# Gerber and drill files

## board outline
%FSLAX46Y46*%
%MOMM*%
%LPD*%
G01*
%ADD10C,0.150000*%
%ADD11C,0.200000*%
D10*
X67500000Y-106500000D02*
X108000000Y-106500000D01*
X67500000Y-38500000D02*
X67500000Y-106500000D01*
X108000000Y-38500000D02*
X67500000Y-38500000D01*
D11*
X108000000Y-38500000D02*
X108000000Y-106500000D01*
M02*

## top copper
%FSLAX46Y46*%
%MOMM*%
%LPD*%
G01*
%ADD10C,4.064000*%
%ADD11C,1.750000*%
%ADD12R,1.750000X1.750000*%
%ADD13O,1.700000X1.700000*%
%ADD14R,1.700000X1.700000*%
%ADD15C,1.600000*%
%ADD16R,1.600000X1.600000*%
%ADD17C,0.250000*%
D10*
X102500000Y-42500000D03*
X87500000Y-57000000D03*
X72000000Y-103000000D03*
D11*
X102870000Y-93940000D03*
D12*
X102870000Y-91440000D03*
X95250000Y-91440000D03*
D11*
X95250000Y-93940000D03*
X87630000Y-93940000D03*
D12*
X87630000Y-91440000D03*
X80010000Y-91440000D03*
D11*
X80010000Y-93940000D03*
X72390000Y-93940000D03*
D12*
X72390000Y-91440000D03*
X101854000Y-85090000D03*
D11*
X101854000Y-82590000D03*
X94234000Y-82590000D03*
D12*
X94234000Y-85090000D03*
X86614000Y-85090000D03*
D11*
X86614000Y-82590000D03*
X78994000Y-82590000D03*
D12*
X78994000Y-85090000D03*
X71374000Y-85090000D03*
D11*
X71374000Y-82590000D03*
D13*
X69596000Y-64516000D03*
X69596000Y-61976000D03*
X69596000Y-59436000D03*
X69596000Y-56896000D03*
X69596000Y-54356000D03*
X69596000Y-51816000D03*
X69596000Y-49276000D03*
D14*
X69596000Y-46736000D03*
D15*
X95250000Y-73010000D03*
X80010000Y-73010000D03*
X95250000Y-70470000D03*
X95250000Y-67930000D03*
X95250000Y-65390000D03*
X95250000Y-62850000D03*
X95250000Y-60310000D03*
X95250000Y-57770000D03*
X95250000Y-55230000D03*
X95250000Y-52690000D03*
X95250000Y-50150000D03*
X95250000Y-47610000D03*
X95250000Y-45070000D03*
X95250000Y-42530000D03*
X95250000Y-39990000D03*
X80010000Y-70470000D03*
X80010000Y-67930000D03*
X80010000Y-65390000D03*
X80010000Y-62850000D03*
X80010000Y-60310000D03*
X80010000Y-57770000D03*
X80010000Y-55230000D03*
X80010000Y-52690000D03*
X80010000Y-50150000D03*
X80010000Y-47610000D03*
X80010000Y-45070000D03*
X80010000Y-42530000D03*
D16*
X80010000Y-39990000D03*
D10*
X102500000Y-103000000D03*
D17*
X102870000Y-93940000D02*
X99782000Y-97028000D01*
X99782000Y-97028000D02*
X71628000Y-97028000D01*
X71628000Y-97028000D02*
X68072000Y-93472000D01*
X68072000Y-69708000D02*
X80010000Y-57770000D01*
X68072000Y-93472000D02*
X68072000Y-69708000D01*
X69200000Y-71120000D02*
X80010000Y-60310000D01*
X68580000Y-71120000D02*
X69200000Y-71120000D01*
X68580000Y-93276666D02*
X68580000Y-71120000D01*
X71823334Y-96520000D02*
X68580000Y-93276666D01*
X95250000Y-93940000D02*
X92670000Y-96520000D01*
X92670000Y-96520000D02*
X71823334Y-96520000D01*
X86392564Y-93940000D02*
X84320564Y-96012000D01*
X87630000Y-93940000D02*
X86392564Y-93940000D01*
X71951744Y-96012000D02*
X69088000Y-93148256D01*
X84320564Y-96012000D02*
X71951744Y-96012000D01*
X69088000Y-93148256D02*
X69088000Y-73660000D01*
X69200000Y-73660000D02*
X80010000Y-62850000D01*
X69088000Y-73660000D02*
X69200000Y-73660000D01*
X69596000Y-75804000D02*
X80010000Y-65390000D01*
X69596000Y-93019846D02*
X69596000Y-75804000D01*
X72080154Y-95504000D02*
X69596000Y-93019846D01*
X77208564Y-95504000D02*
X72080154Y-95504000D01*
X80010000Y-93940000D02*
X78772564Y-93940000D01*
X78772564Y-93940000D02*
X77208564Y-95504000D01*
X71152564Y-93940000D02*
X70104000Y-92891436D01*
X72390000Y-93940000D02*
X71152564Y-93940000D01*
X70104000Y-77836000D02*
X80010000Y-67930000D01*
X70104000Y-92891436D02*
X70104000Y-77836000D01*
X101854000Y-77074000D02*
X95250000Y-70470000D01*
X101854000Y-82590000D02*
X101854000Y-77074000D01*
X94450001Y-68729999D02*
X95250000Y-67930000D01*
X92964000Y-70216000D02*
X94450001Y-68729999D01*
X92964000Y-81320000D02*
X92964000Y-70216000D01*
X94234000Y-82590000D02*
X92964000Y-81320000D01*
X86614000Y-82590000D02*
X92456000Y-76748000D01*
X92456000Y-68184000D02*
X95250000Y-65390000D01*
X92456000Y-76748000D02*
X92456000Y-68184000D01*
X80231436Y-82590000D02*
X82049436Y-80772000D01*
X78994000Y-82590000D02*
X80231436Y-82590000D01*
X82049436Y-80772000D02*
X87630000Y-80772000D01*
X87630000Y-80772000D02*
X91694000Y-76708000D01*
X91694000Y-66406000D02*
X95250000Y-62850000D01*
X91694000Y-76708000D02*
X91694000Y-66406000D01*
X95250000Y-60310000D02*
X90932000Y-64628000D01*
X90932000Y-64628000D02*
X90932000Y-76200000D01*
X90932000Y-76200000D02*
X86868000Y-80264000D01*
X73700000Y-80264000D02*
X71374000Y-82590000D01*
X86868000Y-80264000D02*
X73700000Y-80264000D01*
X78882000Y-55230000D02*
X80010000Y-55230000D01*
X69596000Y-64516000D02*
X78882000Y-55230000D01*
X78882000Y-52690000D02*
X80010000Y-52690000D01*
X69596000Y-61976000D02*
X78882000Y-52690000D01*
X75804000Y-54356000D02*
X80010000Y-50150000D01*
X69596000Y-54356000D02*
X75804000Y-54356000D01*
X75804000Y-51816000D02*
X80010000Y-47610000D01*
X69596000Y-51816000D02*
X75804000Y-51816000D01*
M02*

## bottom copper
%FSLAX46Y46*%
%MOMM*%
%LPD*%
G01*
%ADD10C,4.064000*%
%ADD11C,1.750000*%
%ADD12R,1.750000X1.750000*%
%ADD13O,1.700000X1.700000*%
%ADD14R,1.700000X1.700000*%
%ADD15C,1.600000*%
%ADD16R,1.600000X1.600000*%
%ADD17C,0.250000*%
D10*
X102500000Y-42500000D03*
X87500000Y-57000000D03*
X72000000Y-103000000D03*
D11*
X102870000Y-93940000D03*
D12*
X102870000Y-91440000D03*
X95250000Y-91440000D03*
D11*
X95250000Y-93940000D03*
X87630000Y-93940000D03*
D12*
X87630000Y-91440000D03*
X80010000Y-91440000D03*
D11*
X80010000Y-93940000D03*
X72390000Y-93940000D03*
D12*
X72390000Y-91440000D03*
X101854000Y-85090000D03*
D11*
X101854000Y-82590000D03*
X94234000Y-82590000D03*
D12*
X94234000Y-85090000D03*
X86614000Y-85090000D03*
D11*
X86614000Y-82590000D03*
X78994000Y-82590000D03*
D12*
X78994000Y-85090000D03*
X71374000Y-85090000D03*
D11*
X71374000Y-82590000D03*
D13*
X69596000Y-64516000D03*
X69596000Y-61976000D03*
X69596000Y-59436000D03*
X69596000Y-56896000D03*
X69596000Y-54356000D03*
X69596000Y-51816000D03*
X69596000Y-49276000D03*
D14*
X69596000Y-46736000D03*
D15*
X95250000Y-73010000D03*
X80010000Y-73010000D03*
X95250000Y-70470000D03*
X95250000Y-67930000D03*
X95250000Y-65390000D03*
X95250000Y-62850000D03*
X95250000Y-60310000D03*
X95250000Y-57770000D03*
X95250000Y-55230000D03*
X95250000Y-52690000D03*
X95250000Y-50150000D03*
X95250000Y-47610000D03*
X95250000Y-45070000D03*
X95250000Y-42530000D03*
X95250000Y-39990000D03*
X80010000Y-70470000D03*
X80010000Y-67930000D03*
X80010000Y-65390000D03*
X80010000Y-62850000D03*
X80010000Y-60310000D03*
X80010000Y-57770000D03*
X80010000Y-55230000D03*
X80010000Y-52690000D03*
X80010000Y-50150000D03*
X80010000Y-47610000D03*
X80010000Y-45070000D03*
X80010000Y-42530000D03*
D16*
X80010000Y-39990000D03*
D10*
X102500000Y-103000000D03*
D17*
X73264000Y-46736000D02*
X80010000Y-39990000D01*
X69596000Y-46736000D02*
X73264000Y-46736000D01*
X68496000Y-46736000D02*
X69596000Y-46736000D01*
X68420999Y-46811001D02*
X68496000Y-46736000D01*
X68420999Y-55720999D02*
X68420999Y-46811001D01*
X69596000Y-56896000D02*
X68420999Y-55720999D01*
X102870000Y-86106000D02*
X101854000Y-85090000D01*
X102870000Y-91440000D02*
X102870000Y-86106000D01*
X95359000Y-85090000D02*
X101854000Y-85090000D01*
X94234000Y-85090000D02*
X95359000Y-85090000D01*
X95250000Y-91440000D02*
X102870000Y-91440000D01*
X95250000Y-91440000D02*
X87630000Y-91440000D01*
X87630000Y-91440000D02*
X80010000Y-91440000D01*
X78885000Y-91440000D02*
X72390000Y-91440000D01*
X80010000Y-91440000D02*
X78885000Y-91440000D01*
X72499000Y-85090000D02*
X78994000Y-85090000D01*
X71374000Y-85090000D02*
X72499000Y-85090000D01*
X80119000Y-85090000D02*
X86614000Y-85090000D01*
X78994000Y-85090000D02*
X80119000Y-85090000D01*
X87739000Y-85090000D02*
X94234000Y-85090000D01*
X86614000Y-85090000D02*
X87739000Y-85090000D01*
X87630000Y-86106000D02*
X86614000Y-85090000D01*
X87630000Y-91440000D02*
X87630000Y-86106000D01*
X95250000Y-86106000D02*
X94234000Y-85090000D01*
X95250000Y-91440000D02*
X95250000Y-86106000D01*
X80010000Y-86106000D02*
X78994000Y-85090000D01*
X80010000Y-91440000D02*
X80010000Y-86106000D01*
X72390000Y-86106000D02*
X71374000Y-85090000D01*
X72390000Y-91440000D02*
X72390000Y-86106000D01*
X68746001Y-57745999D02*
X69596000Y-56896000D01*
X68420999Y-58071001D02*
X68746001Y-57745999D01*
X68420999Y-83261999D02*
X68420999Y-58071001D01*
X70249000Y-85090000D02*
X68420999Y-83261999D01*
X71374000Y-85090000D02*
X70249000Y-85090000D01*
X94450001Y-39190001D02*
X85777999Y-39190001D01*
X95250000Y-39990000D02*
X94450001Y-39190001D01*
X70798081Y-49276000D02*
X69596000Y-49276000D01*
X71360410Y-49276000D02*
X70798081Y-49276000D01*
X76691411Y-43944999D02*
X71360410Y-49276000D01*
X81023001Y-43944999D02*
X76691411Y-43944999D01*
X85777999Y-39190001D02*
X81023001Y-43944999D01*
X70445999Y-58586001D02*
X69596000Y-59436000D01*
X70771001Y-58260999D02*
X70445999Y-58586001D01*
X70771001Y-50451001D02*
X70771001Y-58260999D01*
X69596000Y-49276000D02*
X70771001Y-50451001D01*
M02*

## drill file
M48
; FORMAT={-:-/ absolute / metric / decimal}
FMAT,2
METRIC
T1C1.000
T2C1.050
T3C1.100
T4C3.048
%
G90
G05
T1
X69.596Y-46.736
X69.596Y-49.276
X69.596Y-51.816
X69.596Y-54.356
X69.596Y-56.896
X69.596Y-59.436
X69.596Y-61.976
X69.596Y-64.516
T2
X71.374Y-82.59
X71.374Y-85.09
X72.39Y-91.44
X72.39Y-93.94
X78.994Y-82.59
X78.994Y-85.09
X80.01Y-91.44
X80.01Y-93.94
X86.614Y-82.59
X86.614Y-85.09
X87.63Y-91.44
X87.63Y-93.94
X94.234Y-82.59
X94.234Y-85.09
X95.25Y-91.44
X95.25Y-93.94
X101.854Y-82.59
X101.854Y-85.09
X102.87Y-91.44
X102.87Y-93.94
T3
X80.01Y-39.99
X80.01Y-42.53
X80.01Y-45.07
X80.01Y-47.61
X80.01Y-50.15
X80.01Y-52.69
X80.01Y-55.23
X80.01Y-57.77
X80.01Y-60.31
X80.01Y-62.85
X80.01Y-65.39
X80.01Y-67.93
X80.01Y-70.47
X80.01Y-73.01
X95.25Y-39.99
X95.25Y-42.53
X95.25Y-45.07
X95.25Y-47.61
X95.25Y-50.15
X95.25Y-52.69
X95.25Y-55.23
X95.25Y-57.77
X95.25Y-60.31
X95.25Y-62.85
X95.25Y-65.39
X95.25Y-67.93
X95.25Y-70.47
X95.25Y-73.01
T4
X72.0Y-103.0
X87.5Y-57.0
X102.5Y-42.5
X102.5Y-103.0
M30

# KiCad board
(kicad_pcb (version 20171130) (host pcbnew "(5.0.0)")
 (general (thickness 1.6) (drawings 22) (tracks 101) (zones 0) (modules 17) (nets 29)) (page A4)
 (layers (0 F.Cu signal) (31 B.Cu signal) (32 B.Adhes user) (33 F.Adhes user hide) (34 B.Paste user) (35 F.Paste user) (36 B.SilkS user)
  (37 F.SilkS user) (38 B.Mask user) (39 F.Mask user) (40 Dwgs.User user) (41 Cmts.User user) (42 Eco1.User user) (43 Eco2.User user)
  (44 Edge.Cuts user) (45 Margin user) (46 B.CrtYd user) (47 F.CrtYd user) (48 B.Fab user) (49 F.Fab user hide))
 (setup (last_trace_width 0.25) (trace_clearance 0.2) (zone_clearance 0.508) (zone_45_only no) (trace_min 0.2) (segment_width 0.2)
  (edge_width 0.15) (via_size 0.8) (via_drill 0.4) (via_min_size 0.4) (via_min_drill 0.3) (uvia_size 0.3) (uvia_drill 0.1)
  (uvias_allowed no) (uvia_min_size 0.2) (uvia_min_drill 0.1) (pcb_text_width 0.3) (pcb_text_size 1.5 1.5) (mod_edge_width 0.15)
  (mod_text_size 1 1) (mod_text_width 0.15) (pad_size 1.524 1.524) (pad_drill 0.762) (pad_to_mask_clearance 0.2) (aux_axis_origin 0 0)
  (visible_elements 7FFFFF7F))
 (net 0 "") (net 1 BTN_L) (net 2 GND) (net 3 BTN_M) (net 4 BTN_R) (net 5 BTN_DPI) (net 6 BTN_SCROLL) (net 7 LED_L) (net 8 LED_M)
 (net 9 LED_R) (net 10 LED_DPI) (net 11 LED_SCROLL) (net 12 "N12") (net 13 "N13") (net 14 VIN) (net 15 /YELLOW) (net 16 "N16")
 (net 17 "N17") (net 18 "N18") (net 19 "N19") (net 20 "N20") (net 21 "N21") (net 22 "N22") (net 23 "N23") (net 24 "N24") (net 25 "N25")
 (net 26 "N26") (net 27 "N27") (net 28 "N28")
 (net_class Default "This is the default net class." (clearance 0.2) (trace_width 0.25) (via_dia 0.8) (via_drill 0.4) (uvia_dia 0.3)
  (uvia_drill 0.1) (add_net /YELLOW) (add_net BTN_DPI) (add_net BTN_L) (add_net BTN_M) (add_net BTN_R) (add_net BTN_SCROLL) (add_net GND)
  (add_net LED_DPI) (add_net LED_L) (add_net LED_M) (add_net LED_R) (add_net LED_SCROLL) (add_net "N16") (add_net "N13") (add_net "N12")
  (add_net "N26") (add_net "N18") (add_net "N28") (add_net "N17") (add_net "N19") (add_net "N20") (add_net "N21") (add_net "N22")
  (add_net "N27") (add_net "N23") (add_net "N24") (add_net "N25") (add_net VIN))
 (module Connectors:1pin (layer F.Cu) (at 102.5 42.5 90)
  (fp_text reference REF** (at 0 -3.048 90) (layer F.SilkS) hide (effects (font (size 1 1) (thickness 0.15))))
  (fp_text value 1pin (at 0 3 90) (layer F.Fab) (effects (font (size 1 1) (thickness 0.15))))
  (pad 1 thru_hole circle (at 0 0 90) (size 4.064 4.064) (drill 3.048) (layers *.Cu *.Mask)))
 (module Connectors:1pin (layer F.Cu) (at 87.5 57 90)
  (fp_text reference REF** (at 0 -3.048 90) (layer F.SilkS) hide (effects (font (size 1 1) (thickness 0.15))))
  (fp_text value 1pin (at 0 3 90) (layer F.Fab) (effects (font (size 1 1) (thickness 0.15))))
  (pad 1 thru_hole circle (at 0 0 90) (size 4.064 4.064) (drill 3.048) (layers *.Cu *.Mask)))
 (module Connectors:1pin (layer F.Cu) (at 72 103 90)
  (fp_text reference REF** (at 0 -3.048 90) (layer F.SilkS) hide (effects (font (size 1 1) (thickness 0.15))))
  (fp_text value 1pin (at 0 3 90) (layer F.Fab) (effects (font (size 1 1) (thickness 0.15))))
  (pad 1 thru_hole circle (at 0 0 90) (size 4.064 4.064) (drill 3.048) (layers *.Cu *.Mask)))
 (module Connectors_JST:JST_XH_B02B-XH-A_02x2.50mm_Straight (layer F.Cu) (at 102.87 91.44 270)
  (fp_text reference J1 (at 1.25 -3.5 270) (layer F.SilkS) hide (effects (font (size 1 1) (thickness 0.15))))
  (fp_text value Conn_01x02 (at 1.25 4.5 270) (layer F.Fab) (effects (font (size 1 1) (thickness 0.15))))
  (pad 2 thru_hole circle (at 2.5 0 270) (size 1.75 1.75) (drill 1.05) (layers *.Cu *.Mask) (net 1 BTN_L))
  (pad 1 thru_hole rect (at 0 0 270) (size 1.75 1.75) (drill 1.05) (layers *.Cu *.Mask) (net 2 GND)))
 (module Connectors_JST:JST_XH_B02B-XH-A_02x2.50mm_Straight (layer F.Cu) (at 95.25 91.44 270)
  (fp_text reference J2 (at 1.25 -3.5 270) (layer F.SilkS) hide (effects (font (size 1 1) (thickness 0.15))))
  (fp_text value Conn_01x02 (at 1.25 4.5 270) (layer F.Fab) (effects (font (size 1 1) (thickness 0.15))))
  (pad 1 thru_hole rect (at 0 0 270) (size 1.75 1.75) (drill 1.05) (layers *.Cu *.Mask) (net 2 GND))
  (pad 2 thru_hole circle (at 2.5 0 270) (size 1.75 1.75) (drill 1.05) (layers *.Cu *.Mask) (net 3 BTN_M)))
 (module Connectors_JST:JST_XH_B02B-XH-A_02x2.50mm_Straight (layer F.Cu) (at 87.63 91.44 270)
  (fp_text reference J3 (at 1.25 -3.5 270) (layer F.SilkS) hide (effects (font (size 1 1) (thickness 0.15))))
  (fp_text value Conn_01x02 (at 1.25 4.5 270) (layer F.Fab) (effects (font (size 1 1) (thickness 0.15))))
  (pad 2 thru_hole circle (at 2.5 0 270) (size 1.75 1.75) (drill 1.05) (layers *.Cu *.Mask) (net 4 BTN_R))
  (pad 1 thru_hole rect (at 0 0 270) (size 1.75 1.75) (drill 1.05) (layers *.Cu *.Mask) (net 2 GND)))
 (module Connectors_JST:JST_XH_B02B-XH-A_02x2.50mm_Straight (layer F.Cu) (at 80.01 91.44 270)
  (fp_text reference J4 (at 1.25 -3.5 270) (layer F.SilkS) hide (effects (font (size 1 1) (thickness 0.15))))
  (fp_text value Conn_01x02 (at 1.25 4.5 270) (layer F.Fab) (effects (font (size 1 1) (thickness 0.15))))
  (pad 1 thru_hole rect (at 0 0 270) (size 1.75 1.75) (drill 1.05) (layers *.Cu *.Mask) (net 2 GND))
  (pad 2 thru_hole circle (at 2.5 0 270) (size 1.75 1.75) (drill 1.05) (layers *.Cu *.Mask) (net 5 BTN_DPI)))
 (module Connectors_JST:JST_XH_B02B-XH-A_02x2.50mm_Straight (layer F.Cu) (at 72.39 91.44 270)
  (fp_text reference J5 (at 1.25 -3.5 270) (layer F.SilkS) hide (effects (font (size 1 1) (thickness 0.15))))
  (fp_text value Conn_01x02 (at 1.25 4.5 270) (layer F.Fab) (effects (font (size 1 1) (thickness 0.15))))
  (pad 2 thru_hole circle (at 2.5 0 270) (size 1.75 1.75) (drill 1.05) (layers *.Cu *.Mask) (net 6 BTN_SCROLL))
  (pad 1 thru_hole rect (at 0 0 270) (size 1.75 1.75) (drill 1.05) (layers *.Cu *.Mask) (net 2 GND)))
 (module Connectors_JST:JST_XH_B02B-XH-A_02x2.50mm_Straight (layer F.Cu) (at 101.854 85.09 90)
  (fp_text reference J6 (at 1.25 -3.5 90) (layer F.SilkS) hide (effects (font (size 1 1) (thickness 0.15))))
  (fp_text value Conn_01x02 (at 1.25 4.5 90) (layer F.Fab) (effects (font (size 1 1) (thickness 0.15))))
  (pad 1 thru_hole rect (at 0 0 90) (size 1.75 1.75) (drill 1.05) (layers *.Cu *.Mask) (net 2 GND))
  (pad 2 thru_hole circle (at 2.5 0 90) (size 1.75 1.75) (drill 1.05) (layers *.Cu *.Mask) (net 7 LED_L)))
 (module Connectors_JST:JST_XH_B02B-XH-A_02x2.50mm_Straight (layer F.Cu) (at 94.234 85.09 90)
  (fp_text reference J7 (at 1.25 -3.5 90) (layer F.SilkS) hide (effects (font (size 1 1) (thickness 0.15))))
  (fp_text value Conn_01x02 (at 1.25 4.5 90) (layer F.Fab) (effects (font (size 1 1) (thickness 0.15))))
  (pad 2 thru_hole circle (at 2.5 0 90) (size 1.75 1.75) (drill 1.05) (layers *.Cu *.Mask) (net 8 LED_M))
  (pad 1 thru_hole rect (at 0 0 90) (size 1.75 1.75) (drill 1.05) (layers *.Cu *.Mask) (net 2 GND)))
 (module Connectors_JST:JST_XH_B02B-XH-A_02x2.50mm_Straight (layer F.Cu) (at 86.614 85.09 90)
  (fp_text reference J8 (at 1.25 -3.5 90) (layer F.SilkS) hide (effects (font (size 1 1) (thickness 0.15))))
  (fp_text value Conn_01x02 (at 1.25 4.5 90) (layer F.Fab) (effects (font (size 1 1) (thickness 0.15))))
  (pad 1 thru_hole rect (at 0 0 90) (size 1.75 1.75) (drill 1.05) (layers *.Cu *.Mask) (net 2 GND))
  (pad 2 thru_hole circle (at 2.5 0 90) (size 1.75 1.75) (drill 1.05) (layers *.Cu *.Mask) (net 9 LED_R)))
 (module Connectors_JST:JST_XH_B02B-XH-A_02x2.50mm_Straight (layer F.Cu) (at 78.994 85.09 90)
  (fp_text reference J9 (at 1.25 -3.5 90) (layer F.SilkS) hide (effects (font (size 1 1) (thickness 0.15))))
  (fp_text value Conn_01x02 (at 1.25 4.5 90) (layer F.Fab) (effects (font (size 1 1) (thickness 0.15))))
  (pad 2 thru_hole circle (at 2.5 0 90) (size 1.75 1.75) (drill 1.05) (layers *.Cu *.Mask) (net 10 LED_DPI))
  (pad 1 thru_hole rect (at 0 0 90) (size 1.75 1.75) (drill 1.05) (layers *.Cu *.Mask) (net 2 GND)))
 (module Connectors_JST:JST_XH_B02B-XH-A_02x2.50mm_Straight (layer F.Cu) (at 71.374 85.09 90)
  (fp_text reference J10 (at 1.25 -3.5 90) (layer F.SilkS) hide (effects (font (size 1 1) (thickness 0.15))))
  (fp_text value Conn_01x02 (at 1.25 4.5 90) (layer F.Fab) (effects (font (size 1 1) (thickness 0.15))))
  (pad 1 thru_hole rect (at 0 0 90) (size 1.75 1.75) (drill 1.05) (layers *.Cu *.Mask) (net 2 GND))
  (pad 2 thru_hole circle (at 2.5 0 90) (size 1.75 1.75) (drill 1.05) (layers *.Cu *.Mask) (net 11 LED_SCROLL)))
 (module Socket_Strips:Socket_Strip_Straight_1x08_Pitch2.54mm (layer F.Cu) (at 69.596 46.736)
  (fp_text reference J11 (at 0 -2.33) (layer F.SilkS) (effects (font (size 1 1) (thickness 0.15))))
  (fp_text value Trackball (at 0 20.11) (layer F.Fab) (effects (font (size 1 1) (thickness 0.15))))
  (pad 8 thru_hole oval (at 0 17.78) (size 1.7 1.7) (drill 1) (layers *.Cu *.Mask) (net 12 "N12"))
  (pad 7 thru_hole oval (at 0 15.24) (size 1.7 1.7) (drill 1) (layers *.Cu *.Mask) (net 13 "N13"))
  (pad 6 thru_hole oval (at 0 12.7) (size 1.7 1.7) (drill 1) (layers *.Cu *.Mask) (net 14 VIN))
  (pad 5 thru_hole oval (at 0 10.16) (size 1.7 1.7) (drill 1) (layers *.Cu *.Mask) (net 2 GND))
  (pad 4 thru_hole oval (at 0 7.62) (size 1.7 1.7) (drill 1) (layers *.Cu *.Mask) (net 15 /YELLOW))
  (pad 3 thru_hole oval (at 0 5.08) (size 1.7 1.7) (drill 1) (layers *.Cu *.Mask) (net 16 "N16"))
  (pad 2 thru_hole oval (at 0 2.54) (size 1.7 1.7) (drill 1) (layers *.Cu *.Mask) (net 14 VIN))
  (pad 1 thru_hole rect (at 0 0) (size 1.7 1.7) (drill 1) (layers *.Cu *.Mask) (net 2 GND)))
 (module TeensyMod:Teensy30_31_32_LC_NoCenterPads (layer F.Cu) (at 87.63 56.5 270)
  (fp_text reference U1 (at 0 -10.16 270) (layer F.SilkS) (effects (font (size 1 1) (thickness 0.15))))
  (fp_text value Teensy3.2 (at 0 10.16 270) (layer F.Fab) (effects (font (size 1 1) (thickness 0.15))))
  (pad 20 thru_hole circle (at 16.51 -7.62 270) (size 1.6 1.6) (drill 1.1) (layers *.Cu *.Mask F.SilkS) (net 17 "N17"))
  (pad 14 thru_hole circle (at 16.51 7.62 270) (size 1.6 1.6) (drill 1.1) (layers *.Cu *.Mask F.SilkS) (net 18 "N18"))
  (pad 21 thru_hole circle (at 13.97 -7.62 270) (size 1.6 1.6) (drill 1.1) (layers *.Cu *.Mask F.SilkS) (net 7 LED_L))
  (pad 22 thru_hole circle (at 11.43 -7.62 270) (size 1.6 1.6) (drill 1.1) (layers *.Cu *.Mask F.SilkS) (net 8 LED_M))
  (pad 23 thru_hole circle (at 8.89 -7.62 270) (size 1.6 1.6) (drill 1.1) (layers *.Cu *.Mask F.SilkS) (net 9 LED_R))
  (pad 24 thru_hole circle (at 6.35 -7.62 270) (size 1.6 1.6) (drill 1.1) (layers *.Cu *.Mask F.SilkS) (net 10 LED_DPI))
  (pad 25 thru_hole circle (at 3.81 -7.62 270) (size 1.6 1.6) (drill 1.1) (layers *.Cu *.Mask F.SilkS) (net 11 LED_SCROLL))
  (pad 26 thru_hole circle (at 1.27 -7.62 270) (size 1.6 1.6) (drill 1.1) (layers *.Cu *.Mask F.SilkS) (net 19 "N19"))
  (pad 27 thru_hole circle (at -1.27 -7.62 270) (size 1.6 1.6) (drill 1.1) (layers *.Cu *.Mask F.SilkS) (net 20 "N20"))
  (pad 28 thru_hole circle (at -3.81 -7.62 270) (size 1.6 1.6) (drill 1.1) (layers *.Cu *.Mask F.SilkS) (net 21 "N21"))
  (pad 29 thru_hole circle (at -6.35 -7.62 270) (size 1.6 1.6) (drill 1.1) (layers *.Cu *.Mask F.SilkS) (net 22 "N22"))
  (pad 30 thru_hole circle (at -8.89 -7.62 270) (size 1.6 1.6) (drill 1.1) (layers *.Cu *.Mask F.SilkS) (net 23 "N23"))
  (pad 31 thru_hole circle (at -11.43 -7.62 270) (size 1.6 1.6) (drill 1.1) (layers *.Cu *.Mask F.SilkS) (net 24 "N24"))
  (pad 32 thru_hole circle (at -13.97 -7.62 270) (size 1.6 1.6) (drill 1.1) (layers *.Cu *.Mask F.SilkS) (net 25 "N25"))
  (pad 33 thru_hole circle (at -16.51 -7.62 270) (size 1.6 1.6) (drill 1.1) (layers *.Cu *.Mask F.SilkS) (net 14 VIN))
  (pad 13 thru_hole circle (at 13.97 7.62 270) (size 1.6 1.6) (drill 1.1) (layers *.Cu *.Mask F.SilkS) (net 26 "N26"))
  (pad 12 thru_hole circle (at 11.43 7.62 270) (size 1.6 1.6) (drill 1.1) (layers *.Cu *.Mask F.SilkS) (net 6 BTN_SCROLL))
  (pad 11 thru_hole circle (at 8.89 7.62 270) (size 1.6 1.6) (drill 1.1) (layers *.Cu *.Mask F.SilkS) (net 5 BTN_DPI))
  (pad 10 thru_hole circle (at 6.35 7.62 270) (size 1.6 1.6) (drill 1.1) (layers *.Cu *.Mask F.SilkS) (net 4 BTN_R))
  (pad 9 thru_hole circle (at 3.81 7.62 270) (size 1.6 1.6) (drill 1.1) (layers *.Cu *.Mask F.SilkS) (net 3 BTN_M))
  (pad 8 thru_hole circle (at 1.27 7.62 270) (size 1.6 1.6) (drill 1.1) (layers *.Cu *.Mask F.SilkS) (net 1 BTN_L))
  (pad 7 thru_hole circle (at -1.27 7.62 270) (size 1.6 1.6) (drill 1.1) (layers *.Cu *.Mask F.SilkS) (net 12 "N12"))
  (pad 6 thru_hole circle (at -3.81 7.62 270) (size 1.6 1.6) (drill 1.1) (layers *.Cu *.Mask F.SilkS) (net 13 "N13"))
  (pad 5 thru_hole circle (at -6.35 7.62 270) (size 1.6 1.6) (drill 1.1) (layers *.Cu *.Mask F.SilkS) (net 15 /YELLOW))
  (pad 4 thru_hole circle (at -8.89 7.62 270) (size 1.6 1.6) (drill 1.1) (layers *.Cu *.Mask F.SilkS) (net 16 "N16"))
  (pad 3 thru_hole circle (at -11.43 7.62 270) (size 1.6 1.6) (drill 1.1) (layers *.Cu *.Mask F.SilkS) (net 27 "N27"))
  (pad 2 thru_hole circle (at -13.97 7.62 270) (size 1.6 1.6) (drill 1.1) (layers *.Cu *.Mask F.SilkS) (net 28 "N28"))
  (pad 1 thru_hole rect (at -16.51 7.62 270) (size 1.6 1.6) (drill 1.1) (layers *.Cu *.Mask F.SilkS) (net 2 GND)))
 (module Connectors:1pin (layer F.Cu) (at 102.5 103 90)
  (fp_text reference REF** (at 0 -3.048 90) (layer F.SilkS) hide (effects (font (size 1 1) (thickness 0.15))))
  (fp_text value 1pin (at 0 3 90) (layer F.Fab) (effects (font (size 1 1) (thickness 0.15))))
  (pad 1 thru_hole circle (at 0 0 90) (size 4.064 4.064) (drill 3.048) (layers *.Cu *.Mask)))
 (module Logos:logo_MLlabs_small (layer B.Cu) (at 87.5 68.5 180)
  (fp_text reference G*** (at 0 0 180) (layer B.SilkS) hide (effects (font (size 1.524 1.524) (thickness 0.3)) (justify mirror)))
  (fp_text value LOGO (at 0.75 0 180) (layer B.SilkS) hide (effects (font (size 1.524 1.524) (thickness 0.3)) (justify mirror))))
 (gr_line (start 67.5 106.5) (end 108 106.5) (layer Edge.Cuts) (width 0.15))
 (gr_line (start 67.5 38.5) (end 67.5 106.5) (layer Edge.Cuts) (width 0.15))
 (gr_line (start 108 38.5) (end 67.5 38.5) (layer Edge.Cuts) (width 0.15))
 (gr_line (start 108 38.5) (end 108 106.5) (layer Edge.Cuts) (width 0.2))
 (segment (start 102.87 93.94) (end 99.782 97.028) (width 0.25) (layer F.Cu) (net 1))
 (segment (start 99.782 97.028) (end 71.628 97.028) (width 0.25) (layer F.Cu) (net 1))
 (segment (start 71.628 97.028) (end 68.072 93.472) (width 0.25) (layer F.Cu) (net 1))
 (segment (start 68.072 69.708) (end 80.01 57.77) (width 0.25) (layer F.Cu) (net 1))
 (segment (start 68.072 93.472) (end 68.072 69.708) (width 0.25) (layer F.Cu) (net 1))
 (segment (start 73.264 46.736) (end 80.01 39.99) (width 0.25) (layer B.Cu) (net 2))
 (segment (start 69.596 46.736) (end 73.264 46.736) (width 0.25) (layer B.Cu) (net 2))
 (segment (start 68.496 46.736) (end 69.596 46.736) (width 0.25) (layer B.Cu) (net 2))
 (segment (start 68.420999 46.811001) (end 68.496 46.736) (width 0.25) (layer B.Cu) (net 2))
 (segment (start 68.420999 55.720999) (end 68.420999 46.811001) (width 0.25) (layer B.Cu) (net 2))
 (segment (start 69.596 56.896) (end 68.420999 55.720999) (width 0.25) (layer B.Cu) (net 2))
 (segment (start 102.87 86.106) (end 101.854 85.09) (width 0.25) (layer B.Cu) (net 2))
 (segment (start 102.87 91.44) (end 102.87 86.106) (width 0.25) (layer B.Cu) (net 2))
 (segment (start 95.359 85.09) (end 101.854 85.09) (width 0.25) (layer B.Cu) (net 2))
 (segment (start 94.234 85.09) (end 95.359 85.09) (width 0.25) (layer B.Cu) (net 2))
 (segment (start 95.25 91.44) (end 102.87 91.44) (width 0.25) (layer B.Cu) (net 2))
 (segment (start 95.25 91.44) (end 87.63 91.44) (width 0.25) (layer B.Cu) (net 2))
 (segment (start 87.63 91.44) (end 80.01 91.44) (width 0.25) (layer B.Cu) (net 2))
 (segment (start 78.885 91.44) (end 72.39 91.44) (width 0.25) (layer B.Cu) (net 2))
 (segment (start 80.01 91.44) (end 78.885 91.44) (width 0.25) (layer B.Cu) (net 2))
 (segment (start 72.499 85.09) (end 78.994 85.09) (width 0.25) (layer B.Cu) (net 2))
 (segment (start 71.374 85.09) (end 72.499 85.09) (width 0.25) (layer B.Cu) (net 2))
 (segment (start 80.119 85.09) (end 86.614 85.09) (width 0.25) (layer B.Cu) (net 2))
 (segment (start 78.994 85.09) (end 80.119 85.09) (width 0.25) (layer B.Cu) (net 2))
 (segment (start 87.739 85.09) (end 94.234 85.09) (width 0.25) (layer B.Cu) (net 2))
 (segment (start 86.614 85.09) (end 87.739 85.09) (width 0.25) (layer B.Cu) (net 2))
 (segment (start 87.63 86.106) (end 86.614 85.09) (width 0.25) (layer B.Cu) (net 2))
 (segment (start 87.63 91.44) (end 87.63 86.106) (width 0.25) (layer B.Cu) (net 2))
 (segment (start 95.25 86.106) (end 94.234 85.09) (width 0.25) (layer B.Cu) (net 2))
 (segment (start 95.25 91.44) (end 95.25 86.106) (width 0.25) (layer B.Cu) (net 2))
 (segment (start 80.01 86.106) (end 78.994 85.09) (width 0.25) (layer B.Cu) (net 2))
 (segment (start 80.01 91.44) (end 80.01 86.106) (width 0.25) (layer B.Cu) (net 2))
 (segment (start 72.39 86.106) (end 71.374 85.09) (width 0.25) (layer B.Cu) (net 2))
 (segment (start 72.39 91.44) (end 72.39 86.106) (width 0.25) (layer B.Cu) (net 2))
 (segment (start 68.746001 57.745999) (end 69.596 56.896) (width 0.25) (layer B.Cu) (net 2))
 (segment (start 68.420999 58.071001) (end 68.746001 57.745999) (width 0.25) (layer B.Cu) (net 2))
 (segment (start 68.420999 83.261999) (end 68.420999 58.071001) (width 0.25) (layer B.Cu) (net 2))
 (segment (start 70.249 85.09) (end 68.420999 83.261999) (width 0.25) (layer B.Cu) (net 2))
 (segment (start 71.374 85.09) (end 70.249 85.09) (width 0.25) (layer B.Cu) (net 2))
 (segment (start 69.2 71.12) (end 80.01 60.31) (width 0.25) (layer F.Cu) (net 3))
 (segment (start 68.58 71.12) (end 69.2 71.12) (width 0.25) (layer F.Cu) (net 3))
 (segment (start 68.58 93.276666) (end 68.58 71.12) (width 0.25) (layer F.Cu) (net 3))
 (segment (start 71.823334 96.52) (end 68.58 93.276666) (width 0.25) (layer F.Cu) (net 3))
 (segment (start 95.25 93.94) (end 92.67 96.52) (width 0.25) (layer F.Cu) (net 3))
 (segment (start 92.67 96.52) (end 71.823334 96.52) (width 0.25) (layer F.Cu) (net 3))
 (segment (start 86.392564 93.94) (end 84.320564 96.012) (width 0.25) (layer F.Cu) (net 4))
 (segment (start 87.63 93.94) (end 86.392564 93.94) (width 0.25) (layer F.Cu) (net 4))
 (segment (start 71.951744 96.012) (end 69.088 93.148256) (width 0.25) (layer F.Cu) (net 4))
 (segment (start 84.320564 96.012) (end 71.951744 96.012) (width 0.25) (layer F.Cu) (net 4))
 (segment (start 69.088 93.148256) (end 69.088 73.66) (width 0.25) (layer F.Cu) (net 4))
 (segment (start 69.2 73.66) (end 80.01 62.85) (width 0.25) (layer F.Cu) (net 4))
 (segment (start 69.088 73.66) (end 69.2 73.66) (width 0.25) (layer F.Cu) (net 4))
 (segment (start 69.596 75.804) (end 80.01 65.39) (width 0.25) (layer F.Cu) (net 5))
 (segment (start 69.596 93.019846) (end 69.596 75.804) (width 0.25) (layer F.Cu) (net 5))
 (segment (start 72.080154 95.504) (end 69.596 93.019846) (width 0.25) (layer F.Cu) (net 5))
 (segment (start 77.208564 95.504) (end 72.080154 95.504) (width 0.25) (layer F.Cu) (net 5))
 (segment (start 80.01 93.94) (end 78.772564 93.94) (width 0.25) (layer F.Cu) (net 5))
 (segment (start 78.772564 93.94) (end 77.208564 95.504) (width 0.25) (layer F.Cu) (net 5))
 (segment (start 71.152564 93.94) (end 70.104 92.891436) (width 0.25) (layer F.Cu) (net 6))
 (segment (start 72.39 93.94) (end 71.152564 93.94) (width 0.25) (layer F.Cu) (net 6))
 (segment (start 70.104 77.836) (end 80.01 67.93) (width 0.25) (layer F.Cu) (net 6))
 (segment (start 70.104 92.891436) (end 70.104 77.836) (width 0.25) (layer F.Cu) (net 6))
 (segment (start 101.854 77.074) (end 95.25 70.47) (width 0.25) (layer F.Cu) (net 7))
 (segment (start 101.854 82.59) (end 101.854 77.074) (width 0.25) (layer F.Cu) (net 7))
 (segment (start 94.450001 68.729999) (end 95.25 67.93) (width 0.25) (layer F.Cu) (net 8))
 (segment (start 92.964 70.216) (end 94.450001 68.729999) (width 0.25) (layer F.Cu) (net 8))
 (segment (start 92.964 81.32) (end 92.964 70.216) (width 0.25) (layer F.Cu) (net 8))
 (segment (start 94.234 82.59) (end 92.964 81.32) (width 0.25) (layer F.Cu) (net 8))
 (segment (start 86.614 82.59) (end 92.456 76.748) (width 0.25) (layer F.Cu) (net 9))
 (segment (start 92.456 68.184) (end 95.25 65.39) (width 0.25) (layer F.Cu) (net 9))
 (segment (start 92.456 76.748) (end 92.456 68.184) (width 0.25) (layer F.Cu) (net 9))
 (segment (start 80.231436 82.59) (end 82.049436 80.772) (width 0.25) (layer F.Cu) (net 10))
 (segment (start 78.994 82.59) (end 80.231436 82.59) (width 0.25) (layer F.Cu) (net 10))
 (segment (start 82.049436 80.772) (end 87.63 80.772) (width 0.25) (layer F.Cu) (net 10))
 (segment (start 87.63 80.772) (end 91.694 76.708) (width 0.25) (layer F.Cu) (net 10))
 (segment (start 91.694 66.406) (end 95.25 62.85) (width 0.25) (layer F.Cu) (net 10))
 (segment (start 91.694 76.708) (end 91.694 66.406) (width 0.25) (layer F.Cu) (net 10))
 (segment (start 95.25 60.31) (end 90.932 64.628) (width 0.25) (layer F.Cu) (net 11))
 (segment (start 90.932 64.628) (end 90.932 76.2) (width 0.25) (layer F.Cu) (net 11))
 (segment (start 90.932 76.2) (end 86.868 80.264) (width 0.25) (layer F.Cu) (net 11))
 (segment (start 73.7 80.264) (end 71.374 82.59) (width 0.25) (layer F.Cu) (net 11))
 (segment (start 86.868 80.264) (end 73.7 80.264) (width 0.25) (layer F.Cu) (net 11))
 (segment (start 78.882 55.23) (end 80.01 55.23) (width 0.25) (layer F.Cu) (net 12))
 (segment (start 69.596 64.516) (end 78.882 55.23) (width 0.25) (layer F.Cu) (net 12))
 (segment (start 78.882 52.69) (end 80.01 52.69) (width 0.25) (layer F.Cu) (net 13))
 (segment (start 69.596 61.976) (end 78.882 52.69) (width 0.25) (layer F.Cu) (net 13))
 (segment (start 75.804 54.356) (end 80.01 50.15) (width 0.25) (layer F.Cu) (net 15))
 (segment (start 69.596 54.356) (end 75.804 54.356) (width 0.25) (layer F.Cu) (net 15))
 (segment (start 75.804 51.816) (end 80.01 47.61) (width 0.25) (layer F.Cu) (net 16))
 (segment (start 69.596 51.816) (end 75.804 51.816) (width 0.25) (layer F.Cu) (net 16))
 (segment (start 94.450001 39.190001) (end 85.777999 39.190001) (width 0.25) (layer B.Cu) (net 14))
 (segment (start 95.25 39.99) (end 94.450001 39.190001) (width 0.25) (layer B.Cu) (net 14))
 (segment (start 70.798081 49.276) (end 69.596 49.276) (width 0.25) (layer B.Cu) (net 14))
 (segment (start 71.36041 49.276) (end 70.798081 49.276) (width 0.25) (layer B.Cu) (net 14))
 (segment (start 76.691411 43.944999) (end 71.36041 49.276) (width 0.25) (layer B.Cu) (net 14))
 (segment (start 81.023001 43.944999) (end 76.691411 43.944999) (width 0.25) (layer B.Cu) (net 14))
 (segment (start 85.777999 39.190001) (end 81.023001 43.944999) (width 0.25) (layer B.Cu) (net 14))
 (segment (start 70.445999 58.586001) (end 69.596 59.436) (width 0.25) (layer B.Cu) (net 14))
 (segment (start 70.771001 58.260999) (end 70.445999 58.586001) (width 0.25) (layer B.Cu) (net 14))
 (segment (start 70.771001 50.451001) (end 70.771001 58.260999) (width 0.25) (layer B.Cu) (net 14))
 (segment (start 69.596 49.276) (end 70.771001 50.451001) (width 0.25) (layer B.Cu) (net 14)))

